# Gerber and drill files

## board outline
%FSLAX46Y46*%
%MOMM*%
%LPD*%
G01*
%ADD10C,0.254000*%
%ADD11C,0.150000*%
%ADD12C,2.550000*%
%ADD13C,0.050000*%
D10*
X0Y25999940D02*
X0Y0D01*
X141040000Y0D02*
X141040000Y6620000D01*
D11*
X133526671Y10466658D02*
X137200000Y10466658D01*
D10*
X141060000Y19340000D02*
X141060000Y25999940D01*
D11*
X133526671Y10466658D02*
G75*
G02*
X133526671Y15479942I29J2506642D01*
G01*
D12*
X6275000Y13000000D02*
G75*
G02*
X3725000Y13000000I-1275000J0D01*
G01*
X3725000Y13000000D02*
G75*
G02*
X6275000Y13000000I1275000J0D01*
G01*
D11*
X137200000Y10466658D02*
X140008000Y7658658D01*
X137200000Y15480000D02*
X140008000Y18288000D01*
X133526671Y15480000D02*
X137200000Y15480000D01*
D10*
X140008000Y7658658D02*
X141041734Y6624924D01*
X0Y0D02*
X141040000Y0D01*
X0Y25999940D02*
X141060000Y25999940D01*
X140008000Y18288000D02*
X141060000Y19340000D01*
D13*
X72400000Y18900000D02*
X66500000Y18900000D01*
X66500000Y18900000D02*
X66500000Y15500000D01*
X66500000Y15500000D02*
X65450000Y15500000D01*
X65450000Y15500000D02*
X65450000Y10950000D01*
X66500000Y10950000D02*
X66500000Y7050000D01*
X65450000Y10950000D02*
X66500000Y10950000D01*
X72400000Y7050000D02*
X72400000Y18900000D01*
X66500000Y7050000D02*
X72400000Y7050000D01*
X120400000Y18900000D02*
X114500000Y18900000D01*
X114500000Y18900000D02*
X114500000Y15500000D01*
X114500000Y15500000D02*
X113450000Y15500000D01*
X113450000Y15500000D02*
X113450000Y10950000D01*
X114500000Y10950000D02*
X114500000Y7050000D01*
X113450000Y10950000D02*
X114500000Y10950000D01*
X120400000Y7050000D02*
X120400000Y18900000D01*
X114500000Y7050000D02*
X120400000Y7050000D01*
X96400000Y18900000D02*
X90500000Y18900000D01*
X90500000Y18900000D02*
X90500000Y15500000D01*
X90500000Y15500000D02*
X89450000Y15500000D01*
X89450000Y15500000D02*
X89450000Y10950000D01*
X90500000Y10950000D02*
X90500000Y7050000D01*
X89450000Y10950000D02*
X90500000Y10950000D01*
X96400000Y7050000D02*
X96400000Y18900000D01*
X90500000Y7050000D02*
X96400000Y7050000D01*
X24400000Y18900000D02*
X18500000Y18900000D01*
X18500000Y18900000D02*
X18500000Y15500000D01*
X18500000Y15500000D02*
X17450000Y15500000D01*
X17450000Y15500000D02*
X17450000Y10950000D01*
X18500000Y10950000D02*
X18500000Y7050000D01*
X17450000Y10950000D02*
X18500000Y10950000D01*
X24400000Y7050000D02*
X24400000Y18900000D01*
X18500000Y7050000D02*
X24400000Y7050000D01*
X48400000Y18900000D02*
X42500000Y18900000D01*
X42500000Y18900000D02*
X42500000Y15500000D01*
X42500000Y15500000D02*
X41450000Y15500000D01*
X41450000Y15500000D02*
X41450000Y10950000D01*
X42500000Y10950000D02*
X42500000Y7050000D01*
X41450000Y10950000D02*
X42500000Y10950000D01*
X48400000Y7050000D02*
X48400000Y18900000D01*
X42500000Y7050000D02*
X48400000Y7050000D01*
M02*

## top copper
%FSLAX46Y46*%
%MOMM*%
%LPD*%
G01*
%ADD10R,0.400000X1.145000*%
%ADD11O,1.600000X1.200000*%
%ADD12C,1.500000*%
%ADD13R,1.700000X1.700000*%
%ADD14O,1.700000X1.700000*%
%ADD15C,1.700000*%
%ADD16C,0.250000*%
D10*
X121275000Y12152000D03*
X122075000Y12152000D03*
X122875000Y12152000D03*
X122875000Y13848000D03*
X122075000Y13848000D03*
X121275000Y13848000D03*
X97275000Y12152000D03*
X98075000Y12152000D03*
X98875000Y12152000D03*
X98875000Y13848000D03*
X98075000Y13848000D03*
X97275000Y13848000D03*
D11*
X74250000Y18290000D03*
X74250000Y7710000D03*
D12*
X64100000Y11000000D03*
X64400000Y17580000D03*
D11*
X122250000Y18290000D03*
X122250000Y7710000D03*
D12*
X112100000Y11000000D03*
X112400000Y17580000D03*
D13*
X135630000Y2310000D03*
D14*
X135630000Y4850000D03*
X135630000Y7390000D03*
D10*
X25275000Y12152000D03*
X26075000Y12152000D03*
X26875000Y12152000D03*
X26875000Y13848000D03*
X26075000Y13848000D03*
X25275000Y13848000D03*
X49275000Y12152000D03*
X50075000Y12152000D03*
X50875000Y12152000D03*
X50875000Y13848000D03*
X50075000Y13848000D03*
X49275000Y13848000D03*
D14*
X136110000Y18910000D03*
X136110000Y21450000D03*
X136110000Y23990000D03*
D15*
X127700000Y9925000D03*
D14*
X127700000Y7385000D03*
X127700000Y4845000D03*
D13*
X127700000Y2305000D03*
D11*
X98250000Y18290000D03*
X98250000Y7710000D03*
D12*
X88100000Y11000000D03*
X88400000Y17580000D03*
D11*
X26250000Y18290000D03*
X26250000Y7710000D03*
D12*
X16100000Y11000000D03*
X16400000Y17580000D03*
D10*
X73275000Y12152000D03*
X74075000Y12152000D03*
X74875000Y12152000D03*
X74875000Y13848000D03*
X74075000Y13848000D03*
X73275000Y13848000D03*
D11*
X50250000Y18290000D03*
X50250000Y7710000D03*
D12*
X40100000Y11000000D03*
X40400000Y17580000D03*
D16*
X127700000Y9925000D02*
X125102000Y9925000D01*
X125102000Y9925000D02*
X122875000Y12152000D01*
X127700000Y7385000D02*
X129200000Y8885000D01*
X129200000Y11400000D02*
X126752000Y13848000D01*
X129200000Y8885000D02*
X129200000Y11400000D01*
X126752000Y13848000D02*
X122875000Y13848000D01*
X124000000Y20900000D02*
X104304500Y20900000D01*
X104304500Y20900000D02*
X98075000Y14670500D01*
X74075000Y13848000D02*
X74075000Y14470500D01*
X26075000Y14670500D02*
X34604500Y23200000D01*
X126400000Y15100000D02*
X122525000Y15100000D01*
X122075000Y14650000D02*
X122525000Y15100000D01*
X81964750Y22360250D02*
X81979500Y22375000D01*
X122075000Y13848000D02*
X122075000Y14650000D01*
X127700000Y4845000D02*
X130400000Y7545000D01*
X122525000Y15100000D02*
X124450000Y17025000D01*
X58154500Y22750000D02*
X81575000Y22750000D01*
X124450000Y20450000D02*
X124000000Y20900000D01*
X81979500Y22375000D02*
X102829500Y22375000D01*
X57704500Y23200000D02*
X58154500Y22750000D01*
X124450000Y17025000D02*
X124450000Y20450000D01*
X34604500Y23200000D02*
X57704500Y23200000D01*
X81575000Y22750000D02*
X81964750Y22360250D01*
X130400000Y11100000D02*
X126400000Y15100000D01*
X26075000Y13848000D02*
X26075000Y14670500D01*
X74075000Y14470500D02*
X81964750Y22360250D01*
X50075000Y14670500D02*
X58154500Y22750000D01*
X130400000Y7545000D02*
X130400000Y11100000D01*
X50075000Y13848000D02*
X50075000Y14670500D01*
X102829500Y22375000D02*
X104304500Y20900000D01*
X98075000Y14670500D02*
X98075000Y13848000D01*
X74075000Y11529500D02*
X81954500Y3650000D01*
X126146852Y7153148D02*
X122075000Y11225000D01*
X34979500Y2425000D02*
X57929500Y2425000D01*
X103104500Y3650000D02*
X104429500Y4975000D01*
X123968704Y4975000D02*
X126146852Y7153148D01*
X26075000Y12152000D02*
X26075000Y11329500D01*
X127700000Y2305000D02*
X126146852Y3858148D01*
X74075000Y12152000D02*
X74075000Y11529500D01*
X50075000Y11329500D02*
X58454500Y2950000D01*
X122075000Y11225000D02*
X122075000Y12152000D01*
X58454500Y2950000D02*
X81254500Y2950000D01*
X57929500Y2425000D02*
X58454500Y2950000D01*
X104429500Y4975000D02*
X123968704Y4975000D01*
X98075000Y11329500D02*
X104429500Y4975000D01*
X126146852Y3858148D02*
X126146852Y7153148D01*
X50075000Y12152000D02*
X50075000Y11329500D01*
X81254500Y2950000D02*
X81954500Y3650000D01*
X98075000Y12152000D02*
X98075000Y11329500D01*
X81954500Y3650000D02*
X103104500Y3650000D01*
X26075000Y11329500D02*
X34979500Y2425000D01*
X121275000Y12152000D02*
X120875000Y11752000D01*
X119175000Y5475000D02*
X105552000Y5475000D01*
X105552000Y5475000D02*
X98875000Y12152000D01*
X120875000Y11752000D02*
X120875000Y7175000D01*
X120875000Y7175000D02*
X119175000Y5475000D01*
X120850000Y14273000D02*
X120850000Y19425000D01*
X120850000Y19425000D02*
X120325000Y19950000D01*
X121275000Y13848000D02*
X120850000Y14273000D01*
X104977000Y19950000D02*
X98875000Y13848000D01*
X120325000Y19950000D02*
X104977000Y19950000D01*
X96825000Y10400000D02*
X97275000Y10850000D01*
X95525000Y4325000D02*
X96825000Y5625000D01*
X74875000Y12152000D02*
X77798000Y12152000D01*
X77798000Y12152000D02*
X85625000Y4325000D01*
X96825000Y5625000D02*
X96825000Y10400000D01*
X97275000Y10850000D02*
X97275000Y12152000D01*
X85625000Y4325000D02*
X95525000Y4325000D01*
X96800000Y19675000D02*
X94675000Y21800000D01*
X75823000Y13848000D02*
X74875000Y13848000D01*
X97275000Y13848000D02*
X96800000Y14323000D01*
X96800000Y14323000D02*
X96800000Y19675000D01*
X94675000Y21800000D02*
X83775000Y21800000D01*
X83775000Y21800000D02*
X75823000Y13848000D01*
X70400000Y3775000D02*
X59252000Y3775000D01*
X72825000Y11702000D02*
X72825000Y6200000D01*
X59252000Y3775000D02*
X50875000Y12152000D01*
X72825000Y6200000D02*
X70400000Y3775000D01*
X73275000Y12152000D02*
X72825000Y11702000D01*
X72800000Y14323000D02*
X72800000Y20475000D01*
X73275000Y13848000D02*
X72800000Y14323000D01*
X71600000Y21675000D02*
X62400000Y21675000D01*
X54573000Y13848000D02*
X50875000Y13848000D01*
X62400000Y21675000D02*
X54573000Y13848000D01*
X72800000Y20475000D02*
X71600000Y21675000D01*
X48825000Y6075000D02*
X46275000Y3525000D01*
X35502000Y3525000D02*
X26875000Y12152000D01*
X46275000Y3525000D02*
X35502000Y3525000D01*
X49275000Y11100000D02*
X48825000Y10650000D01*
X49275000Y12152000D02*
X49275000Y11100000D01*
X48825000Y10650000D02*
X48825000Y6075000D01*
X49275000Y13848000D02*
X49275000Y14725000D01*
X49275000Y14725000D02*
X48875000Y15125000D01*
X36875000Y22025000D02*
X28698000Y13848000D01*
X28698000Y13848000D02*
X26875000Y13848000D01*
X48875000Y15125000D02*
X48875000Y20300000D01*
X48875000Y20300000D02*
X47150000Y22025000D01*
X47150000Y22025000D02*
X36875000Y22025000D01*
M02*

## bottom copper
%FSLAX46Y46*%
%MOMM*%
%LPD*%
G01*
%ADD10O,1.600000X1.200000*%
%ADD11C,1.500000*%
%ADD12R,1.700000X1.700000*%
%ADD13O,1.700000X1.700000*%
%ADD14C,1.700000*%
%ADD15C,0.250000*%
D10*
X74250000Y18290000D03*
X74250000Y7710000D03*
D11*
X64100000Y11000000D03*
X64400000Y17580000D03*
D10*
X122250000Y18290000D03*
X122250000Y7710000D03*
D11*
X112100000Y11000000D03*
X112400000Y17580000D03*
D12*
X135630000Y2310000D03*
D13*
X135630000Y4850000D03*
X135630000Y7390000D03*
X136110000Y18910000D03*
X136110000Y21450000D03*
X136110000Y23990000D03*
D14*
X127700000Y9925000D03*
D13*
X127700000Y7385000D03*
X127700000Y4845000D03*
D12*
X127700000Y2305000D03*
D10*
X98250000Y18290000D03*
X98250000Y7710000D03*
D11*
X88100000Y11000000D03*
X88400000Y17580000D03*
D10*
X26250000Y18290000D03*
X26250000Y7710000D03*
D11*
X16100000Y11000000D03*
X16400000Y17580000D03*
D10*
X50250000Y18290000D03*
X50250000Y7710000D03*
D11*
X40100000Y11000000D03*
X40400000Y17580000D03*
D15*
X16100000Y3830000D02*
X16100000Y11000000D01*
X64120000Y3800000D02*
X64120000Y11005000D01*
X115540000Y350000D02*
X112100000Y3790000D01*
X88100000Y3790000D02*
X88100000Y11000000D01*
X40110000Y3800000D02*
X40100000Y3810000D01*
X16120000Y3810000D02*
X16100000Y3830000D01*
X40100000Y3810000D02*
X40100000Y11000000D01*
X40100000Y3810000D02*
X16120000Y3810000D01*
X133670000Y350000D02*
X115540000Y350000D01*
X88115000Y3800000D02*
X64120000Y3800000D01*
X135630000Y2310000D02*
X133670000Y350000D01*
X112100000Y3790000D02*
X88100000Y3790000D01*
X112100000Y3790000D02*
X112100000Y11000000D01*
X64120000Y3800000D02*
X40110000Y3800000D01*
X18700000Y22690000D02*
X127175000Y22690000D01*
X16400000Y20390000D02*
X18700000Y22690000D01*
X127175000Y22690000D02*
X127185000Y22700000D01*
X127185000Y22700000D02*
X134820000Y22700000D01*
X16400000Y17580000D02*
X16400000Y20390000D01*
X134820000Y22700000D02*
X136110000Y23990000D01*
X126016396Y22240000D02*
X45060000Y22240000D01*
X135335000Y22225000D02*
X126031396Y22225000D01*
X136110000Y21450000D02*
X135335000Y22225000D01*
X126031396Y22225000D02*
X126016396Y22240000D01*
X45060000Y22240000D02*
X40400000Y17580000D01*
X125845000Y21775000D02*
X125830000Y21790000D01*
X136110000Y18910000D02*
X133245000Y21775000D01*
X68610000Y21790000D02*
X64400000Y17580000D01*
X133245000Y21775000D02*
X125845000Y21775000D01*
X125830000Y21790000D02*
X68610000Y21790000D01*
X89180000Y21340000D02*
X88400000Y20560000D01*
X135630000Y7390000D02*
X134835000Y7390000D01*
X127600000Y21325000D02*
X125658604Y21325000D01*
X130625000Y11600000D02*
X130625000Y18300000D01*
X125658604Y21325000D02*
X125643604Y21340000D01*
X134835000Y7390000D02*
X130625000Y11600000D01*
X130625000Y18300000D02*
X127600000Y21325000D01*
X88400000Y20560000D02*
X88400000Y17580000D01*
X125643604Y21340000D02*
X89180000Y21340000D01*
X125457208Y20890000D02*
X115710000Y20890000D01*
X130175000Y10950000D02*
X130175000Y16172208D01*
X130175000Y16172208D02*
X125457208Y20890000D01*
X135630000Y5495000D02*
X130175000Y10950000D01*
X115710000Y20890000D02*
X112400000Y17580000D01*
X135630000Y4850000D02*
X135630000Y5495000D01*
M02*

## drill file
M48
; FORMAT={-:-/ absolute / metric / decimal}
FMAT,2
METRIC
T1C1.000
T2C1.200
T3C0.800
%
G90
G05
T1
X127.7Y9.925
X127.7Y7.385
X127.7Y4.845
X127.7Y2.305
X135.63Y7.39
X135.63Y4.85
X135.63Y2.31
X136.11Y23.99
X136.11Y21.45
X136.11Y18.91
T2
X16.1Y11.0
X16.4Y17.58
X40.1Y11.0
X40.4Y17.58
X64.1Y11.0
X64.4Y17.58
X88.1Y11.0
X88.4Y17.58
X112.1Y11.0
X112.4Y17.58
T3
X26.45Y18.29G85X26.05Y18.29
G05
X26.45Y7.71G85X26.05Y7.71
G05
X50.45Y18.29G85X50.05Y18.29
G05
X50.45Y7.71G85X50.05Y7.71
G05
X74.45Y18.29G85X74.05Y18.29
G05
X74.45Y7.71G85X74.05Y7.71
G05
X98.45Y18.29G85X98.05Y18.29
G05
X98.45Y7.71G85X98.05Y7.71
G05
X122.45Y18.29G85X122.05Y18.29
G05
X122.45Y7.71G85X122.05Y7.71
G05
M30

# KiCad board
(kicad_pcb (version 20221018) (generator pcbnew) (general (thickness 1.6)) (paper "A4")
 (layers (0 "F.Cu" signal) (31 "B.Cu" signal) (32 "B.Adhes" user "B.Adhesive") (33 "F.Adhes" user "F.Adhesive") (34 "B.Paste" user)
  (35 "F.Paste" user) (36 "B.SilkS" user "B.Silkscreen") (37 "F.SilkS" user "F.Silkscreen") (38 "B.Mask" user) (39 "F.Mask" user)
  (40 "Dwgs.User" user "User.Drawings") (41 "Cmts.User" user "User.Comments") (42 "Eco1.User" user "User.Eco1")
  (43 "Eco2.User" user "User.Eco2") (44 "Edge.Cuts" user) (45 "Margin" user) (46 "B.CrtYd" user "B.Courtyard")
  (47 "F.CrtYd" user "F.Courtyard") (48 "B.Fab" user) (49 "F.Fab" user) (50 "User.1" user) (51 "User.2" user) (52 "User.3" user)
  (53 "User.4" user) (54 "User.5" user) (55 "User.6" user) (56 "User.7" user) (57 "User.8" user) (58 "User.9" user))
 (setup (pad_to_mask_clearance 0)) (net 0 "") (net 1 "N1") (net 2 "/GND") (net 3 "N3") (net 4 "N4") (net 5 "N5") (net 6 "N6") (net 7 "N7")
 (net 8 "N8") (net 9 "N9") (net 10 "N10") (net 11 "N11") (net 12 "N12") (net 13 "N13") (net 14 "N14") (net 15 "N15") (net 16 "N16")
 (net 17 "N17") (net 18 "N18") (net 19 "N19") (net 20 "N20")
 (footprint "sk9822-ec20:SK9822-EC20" (layer "F.Cu") (at 122.075 -13 90)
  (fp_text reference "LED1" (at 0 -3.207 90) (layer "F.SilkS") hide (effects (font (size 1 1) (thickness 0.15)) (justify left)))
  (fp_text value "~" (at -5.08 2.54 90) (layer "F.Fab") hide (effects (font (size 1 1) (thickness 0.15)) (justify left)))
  (pad "1" smd rect (at -0.848 -0.8 90) (size 1.145 0.4) (layers "F.Cu" "F.Paste" "F.Mask") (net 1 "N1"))
  (pad "2" smd rect (at -0.848 0 90) (size 1.145 0.4) (layers "F.Cu" "F.Paste" "F.Mask") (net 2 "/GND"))
  (pad "3" smd rect (at -0.848 0.8 90) (size 1.145 0.4) (layers "F.Cu" "F.Paste" "F.Mask") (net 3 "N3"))
  (pad "4" smd rect (at 0.848 0.8 90) (size 1.145 0.4) (layers "F.Cu" "F.Paste" "F.Mask") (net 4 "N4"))
  (pad "5" smd rect (at 0.848 0 90) (size 1.145 0.4) (layers "F.Cu" "F.Paste" "F.Mask") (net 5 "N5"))
  (pad "6" smd rect (at 0.848 -0.8 90) (size 1.145 0.4) (layers "F.Cu" "F.Paste" "F.Mask") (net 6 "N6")))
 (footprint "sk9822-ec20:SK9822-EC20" (layer "F.Cu") (at 98.075 -13 90)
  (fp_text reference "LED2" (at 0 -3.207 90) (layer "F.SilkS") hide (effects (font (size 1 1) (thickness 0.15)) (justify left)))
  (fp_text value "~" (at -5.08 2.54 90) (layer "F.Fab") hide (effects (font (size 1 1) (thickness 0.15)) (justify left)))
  (pad "1" smd rect (at -0.848 -0.8 90) (size 1.145 0.4) (layers "F.Cu" "F.Paste" "F.Mask") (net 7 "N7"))
  (pad "2" smd rect (at -0.848 0 90) (size 1.145 0.4) (layers "F.Cu" "F.Paste" "F.Mask") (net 2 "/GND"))
  (pad "3" smd rect (at -0.848 0.8 90) (size 1.145 0.4) (layers "F.Cu" "F.Paste" "F.Mask") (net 1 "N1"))
  (pad "4" smd rect (at 0.848 0.8 90) (size 1.145 0.4) (layers "F.Cu" "F.Paste" "F.Mask") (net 6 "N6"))
  (pad "5" smd rect (at 0.848 0 90) (size 1.145 0.4) (layers "F.Cu" "F.Paste" "F.Mask") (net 5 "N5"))
  (pad "6" smd rect (at 0.848 -0.8 90) (size 1.145 0.4) (layers "F.Cu" "F.Paste" "F.Mask") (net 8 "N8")))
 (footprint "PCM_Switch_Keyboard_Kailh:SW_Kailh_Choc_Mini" (layer "F.Cu") (at 69.5 -13 -90)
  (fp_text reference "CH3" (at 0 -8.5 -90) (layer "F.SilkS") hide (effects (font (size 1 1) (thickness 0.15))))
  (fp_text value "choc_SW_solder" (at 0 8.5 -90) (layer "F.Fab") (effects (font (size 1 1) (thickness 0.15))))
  (fp_line (start -5.9 -2.9) (end -5.9 3) (stroke (width 0.05) (type solid)) (layer "Edge.Cuts"))
  (fp_line (start -5.9 3) (end -2.5 3) (stroke (width 0.05) (type solid)) (layer "Edge.Cuts"))
  (fp_line (start -2.5 3) (end -2.5 4.05) (stroke (width 0.05) (type solid)) (layer "Edge.Cuts"))
  (fp_line (start -2.5 4.05) (end 2.05 4.05) (stroke (width 0.05) (type solid)) (layer "Edge.Cuts"))
  (fp_line (start 2.05 3) (end 5.95 3) (stroke (width 0.05) (type solid)) (layer "Edge.Cuts"))
  (fp_line (start 2.05 4.05) (end 2.05 3) (stroke (width 0.05) (type solid)) (layer "Edge.Cuts"))
  (fp_line (start 5.95 -2.9) (end -5.9 -2.9) (stroke (width 0.05) (type solid)) (layer "Edge.Cuts"))
  (fp_line (start 5.95 3) (end 5.95 -2.9) (stroke (width 0.05) (type solid)) (layer "Edge.Cuts"))
  (pad "" np_thru_hole oval (at -5.29 -4.75 270) (size 1.2 1.6) (drill oval 0.8 1.2) (layers "*.Cu" "*.Mask"))
  (pad "" np_thru_hole oval (at 5.29 -4.75 270) (size 1.2 1.6) (drill oval 0.8 1.2) (layers "*.Cu" "*.Mask"))
  (pad "1" thru_hole circle (at 2 5.4 270) (size 1.5 1.5) (drill 1.2) (layers "*.Cu" "*.Mask") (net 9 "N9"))
  (pad "2" thru_hole circle (at -4.58 5.1 270) (size 1.5 1.5) (drill 1.2) (layers "*.Cu" "*.Mask") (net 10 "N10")))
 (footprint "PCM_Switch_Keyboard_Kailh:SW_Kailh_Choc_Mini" (layer "F.Cu") (at 117.5 -13 -90)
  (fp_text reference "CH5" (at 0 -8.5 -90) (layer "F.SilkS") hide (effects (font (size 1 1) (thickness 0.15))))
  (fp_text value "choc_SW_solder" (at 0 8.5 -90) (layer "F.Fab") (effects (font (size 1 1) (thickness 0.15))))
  (fp_line (start -5.9 -2.9) (end -5.9 3) (stroke (width 0.05) (type solid)) (layer "Edge.Cuts"))
  (fp_line (start -5.9 3) (end -2.5 3) (stroke (width 0.05) (type solid)) (layer "Edge.Cuts"))
  (fp_line (start -2.5 3) (end -2.5 4.05) (stroke (width 0.05) (type solid)) (layer "Edge.Cuts"))
  (fp_line (start -2.5 4.05) (end 2.05 4.05) (stroke (width 0.05) (type solid)) (layer "Edge.Cuts"))
  (fp_line (start 2.05 3) (end 5.95 3) (stroke (width 0.05) (type solid)) (layer "Edge.Cuts"))
  (fp_line (start 2.05 4.05) (end 2.05 3) (stroke (width 0.05) (type solid)) (layer "Edge.Cuts"))
  (fp_line (start 5.95 -2.9) (end -5.9 -2.9) (stroke (width 0.05) (type solid)) (layer "Edge.Cuts"))
  (fp_line (start 5.95 3) (end 5.95 -2.9) (stroke (width 0.05) (type solid)) (layer "Edge.Cuts"))
  (pad "" np_thru_hole oval (at -5.29 -4.75 270) (size 1.2 1.6) (drill oval 0.8 1.2) (layers "*.Cu" "*.Mask"))
  (pad "" np_thru_hole oval (at 5.29 -4.75 270) (size 1.2 1.6) (drill oval 0.8 1.2) (layers "*.Cu" "*.Mask"))
  (pad "1" thru_hole circle (at 2 5.4 270) (size 1.5 1.5) (drill 1.2) (layers "*.Cu" "*.Mask") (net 9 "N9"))
  (pad "2" thru_hole circle (at -4.58 5.1 270) (size 1.5 1.5) (drill 1.2) (layers "*.Cu" "*.Mask") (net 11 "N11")))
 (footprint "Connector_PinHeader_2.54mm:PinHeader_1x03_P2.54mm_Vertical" (layer "F.Cu") (at 135.63 -2.31 180)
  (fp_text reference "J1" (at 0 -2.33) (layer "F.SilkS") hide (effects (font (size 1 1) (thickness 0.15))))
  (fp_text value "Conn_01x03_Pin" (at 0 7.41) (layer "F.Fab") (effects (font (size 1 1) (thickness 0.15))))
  (pad "1" thru_hole rect (at 0 0 180) (size 1.7 1.7) (drill 1) (layers "*.Cu" "*.Mask") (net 9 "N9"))
  (pad "2" thru_hole oval (at 0 2.54 180) (size 1.7 1.7) (drill 1) (layers "*.Cu" "*.Mask") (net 11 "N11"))
  (pad "3" thru_hole oval (at 0 5.08 180) (size 1.7 1.7) (drill 1) (layers "*.Cu" "*.Mask") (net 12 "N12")))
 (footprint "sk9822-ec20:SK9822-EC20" (layer "F.Cu") (at 26.075 -13 90)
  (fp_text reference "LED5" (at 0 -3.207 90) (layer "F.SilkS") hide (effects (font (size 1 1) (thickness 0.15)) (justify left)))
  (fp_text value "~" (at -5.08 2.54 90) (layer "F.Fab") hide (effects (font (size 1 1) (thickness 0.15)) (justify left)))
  (pad "1" smd rect (at -0.848 -0.8 90) (size 1.145 0.4) (layers "F.Cu" "F.Paste" "F.Mask") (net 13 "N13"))
  (pad "2" smd rect (at -0.848 0 90) (size 1.145 0.4) (layers "F.Cu" "F.Paste" "F.Mask") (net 2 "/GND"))
  (pad "3" smd rect (at -0.848 0.8 90) (size 1.145 0.4) (layers "F.Cu" "F.Paste" "F.Mask") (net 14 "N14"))
  (pad "4" smd rect (at 0.848 0.8 90) (size 1.145 0.4) (layers "F.Cu" "F.Paste" "F.Mask") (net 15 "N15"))
  (pad "5" smd rect (at 0.848 0 90) (size 1.145 0.4) (layers "F.Cu" "F.Paste" "F.Mask") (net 5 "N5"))
  (pad "6" smd rect (at 0.848 -0.8 90) (size 1.145 0.4) (layers "F.Cu" "F.Paste" "F.Mask") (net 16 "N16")))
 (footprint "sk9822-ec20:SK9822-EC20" (layer "F.Cu") (at 50.075 -13 90)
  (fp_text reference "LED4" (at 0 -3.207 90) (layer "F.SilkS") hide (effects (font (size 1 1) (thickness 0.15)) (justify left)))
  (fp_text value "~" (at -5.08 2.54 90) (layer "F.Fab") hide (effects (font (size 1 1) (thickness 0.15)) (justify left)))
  (pad "1" smd rect (at -0.848 -0.8 90) (size 1.145 0.4) (layers "F.Cu" "F.Paste" "F.Mask") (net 14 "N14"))
  (pad "2" smd rect (at -0.848 0 90) (size 1.145 0.4) (layers "F.Cu" "F.Paste" "F.Mask") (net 2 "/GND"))
  (pad "3" smd rect (at -0.848 0.8 90) (size 1.145 0.4) (layers "F.Cu" "F.Paste" "F.Mask") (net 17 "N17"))
  (pad "4" smd rect (at 0.848 0.8 90) (size 1.145 0.4) (layers "F.Cu" "F.Paste" "F.Mask") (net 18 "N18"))
  (pad "5" smd rect (at 0.848 0 90) (size 1.145 0.4) (layers "F.Cu" "F.Paste" "F.Mask") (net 5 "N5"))
  (pad "6" smd rect (at 0.848 -0.8 90) (size 1.145 0.4) (layers "F.Cu" "F.Paste" "F.Mask") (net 15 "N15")))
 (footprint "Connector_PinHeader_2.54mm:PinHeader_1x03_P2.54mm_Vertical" (layer "F.Cu") (at 136.11 -18.91 180)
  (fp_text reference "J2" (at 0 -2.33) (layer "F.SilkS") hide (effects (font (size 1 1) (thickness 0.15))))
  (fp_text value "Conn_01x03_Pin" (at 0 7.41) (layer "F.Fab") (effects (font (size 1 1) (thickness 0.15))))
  (pad "1" thru_hole oval (at 0 0 180) (size 1.7 1.7) (drill 1) (layers "*.Cu" "*.Mask") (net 10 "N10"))
  (pad "2" thru_hole oval (at 0 2.54 180) (size 1.7 1.7) (drill 1) (layers "*.Cu" "*.Mask") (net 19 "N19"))
  (pad "3" thru_hole oval (at 0 5.08 180) (size 1.7 1.7) (drill 1) (layers "*.Cu" "*.Mask") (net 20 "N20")))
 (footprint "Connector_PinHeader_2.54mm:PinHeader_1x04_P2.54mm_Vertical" (layer "F.Cu") (at 127.7 -9.925)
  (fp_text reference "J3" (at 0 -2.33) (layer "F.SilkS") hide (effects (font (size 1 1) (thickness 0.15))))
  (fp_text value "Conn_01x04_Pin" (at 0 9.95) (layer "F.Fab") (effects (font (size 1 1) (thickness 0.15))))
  (pad "1" thru_hole circle (at 0 0) (size 1.7 1.7) (drill 1) (layers "*.Cu" "*.Mask") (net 3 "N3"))
  (pad "2" thru_hole oval (at 0 2.54) (size 1.7 1.7) (drill 1) (layers "*.Cu" "*.Mask") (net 4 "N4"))
  (pad "3" thru_hole oval (at 0 5.08) (size 1.7 1.7) (drill 1) (layers "*.Cu" "*.Mask") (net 5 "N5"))
  (pad "4" thru_hole rect (at 0 7.62) (size 1.7 1.7) (drill 1) (layers "*.Cu" "*.Mask") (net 2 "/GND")))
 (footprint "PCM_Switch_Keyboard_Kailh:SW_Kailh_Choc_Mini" (layer "F.Cu") (at 93.5 -13 -90)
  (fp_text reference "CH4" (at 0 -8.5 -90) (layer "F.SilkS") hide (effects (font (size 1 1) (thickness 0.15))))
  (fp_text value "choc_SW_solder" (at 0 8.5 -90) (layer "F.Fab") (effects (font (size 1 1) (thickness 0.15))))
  (fp_line (start -5.9 -2.9) (end -5.9 3) (stroke (width 0.05) (type solid)) (layer "Edge.Cuts"))
  (fp_line (start -5.9 3) (end -2.5 3) (stroke (width 0.05) (type solid)) (layer "Edge.Cuts"))
  (fp_line (start -2.5 3) (end -2.5 4.05) (stroke (width 0.05) (type solid)) (layer "Edge.Cuts"))
  (fp_line (start -2.5 4.05) (end 2.05 4.05) (stroke (width 0.05) (type solid)) (layer "Edge.Cuts"))
  (fp_line (start 2.05 3) (end 5.95 3) (stroke (width 0.05) (type solid)) (layer "Edge.Cuts"))
  (fp_line (start 2.05 4.05) (end 2.05 3) (stroke (width 0.05) (type solid)) (layer "Edge.Cuts"))
  (fp_line (start 5.95 -2.9) (end -5.9 -2.9) (stroke (width 0.05) (type solid)) (layer "Edge.Cuts"))
  (fp_line (start 5.95 3) (end 5.95 -2.9) (stroke (width 0.05) (type solid)) (layer "Edge.Cuts"))
  (pad "" np_thru_hole oval (at -5.29 -4.75 270) (size 1.2 1.6) (drill oval 0.8 1.2) (layers "*.Cu" "*.Mask"))
  (pad "" np_thru_hole oval (at 5.29 -4.75 270) (size 1.2 1.6) (drill oval 0.8 1.2) (layers "*.Cu" "*.Mask"))
  (pad "1" thru_hole circle (at 2 5.4 270) (size 1.5 1.5) (drill 1.2) (layers "*.Cu" "*.Mask") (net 9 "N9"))
  (pad "2" thru_hole circle (at -4.58 5.1 270) (size 1.5 1.5) (drill 1.2) (layers "*.Cu" "*.Mask") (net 12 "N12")))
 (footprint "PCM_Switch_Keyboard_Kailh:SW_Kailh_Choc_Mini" (layer "F.Cu") (at 21.5 -13 -90)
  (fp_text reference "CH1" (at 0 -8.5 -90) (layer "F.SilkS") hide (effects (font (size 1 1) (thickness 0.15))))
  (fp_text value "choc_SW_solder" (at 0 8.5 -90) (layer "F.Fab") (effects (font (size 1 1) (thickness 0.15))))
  (fp_line (start -5.9 -2.9) (end -5.9 3) (stroke (width 0.05) (type solid)) (layer "Edge.Cuts"))
  (fp_line (start -5.9 3) (end -2.5 3) (stroke (width 0.05) (type solid)) (layer "Edge.Cuts"))
  (fp_line (start -2.5 3) (end -2.5 4.05) (stroke (width 0.05) (type solid)) (layer "Edge.Cuts"))
  (fp_line (start -2.5 4.05) (end 2.05 4.05) (stroke (width 0.05) (type solid)) (layer "Edge.Cuts"))
  (fp_line (start 2.05 3) (end 5.95 3) (stroke (width 0.05) (type solid)) (layer "Edge.Cuts"))
  (fp_line (start 2.05 4.05) (end 2.05 3) (stroke (width 0.05) (type solid)) (layer "Edge.Cuts"))
  (fp_line (start 5.95 -2.9) (end -5.9 -2.9) (stroke (width 0.05) (type solid)) (layer "Edge.Cuts"))
  (fp_line (start 5.95 3) (end 5.95 -2.9) (stroke (width 0.05) (type solid)) (layer "Edge.Cuts"))
  (pad "" np_thru_hole oval (at -5.29 -4.75 270) (size 1.2 1.6) (drill oval 0.8 1.2) (layers "*.Cu" "*.Mask"))
  (pad "" np_thru_hole oval (at 5.29 -4.75 270) (size 1.2 1.6) (drill oval 0.8 1.2) (layers "*.Cu" "*.Mask"))
  (pad "1" thru_hole circle (at 2 5.4 270) (size 1.5 1.5) (drill 1.2) (layers "*.Cu" "*.Mask") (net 9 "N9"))
  (pad "2" thru_hole circle (at -4.58 5.1 270) (size 1.5 1.5) (drill 1.2) (layers "*.Cu" "*.Mask") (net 20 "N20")))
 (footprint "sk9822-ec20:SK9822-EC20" (layer "F.Cu") (at 74.075 -13 90)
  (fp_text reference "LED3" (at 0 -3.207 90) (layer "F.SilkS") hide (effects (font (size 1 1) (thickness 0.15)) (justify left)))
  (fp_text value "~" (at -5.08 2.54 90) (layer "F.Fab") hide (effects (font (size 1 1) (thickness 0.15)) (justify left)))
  (pad "1" smd rect (at -0.848 -0.8 90) (size 1.145 0.4) (layers "F.Cu" "F.Paste" "F.Mask") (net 17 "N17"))
  (pad "2" smd rect (at -0.848 0 90) (size 1.145 0.4) (layers "F.Cu" "F.Paste" "F.Mask") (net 2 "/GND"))
  (pad "3" smd rect (at -0.848 0.8 90) (size 1.145 0.4) (layers "F.Cu" "F.Paste" "F.Mask") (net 7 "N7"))
  (pad "4" smd rect (at 0.848 0.8 90) (size 1.145 0.4) (layers "F.Cu" "F.Paste" "F.Mask") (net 8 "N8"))
  (pad "5" smd rect (at 0.848 0 90) (size 1.145 0.4) (layers "F.Cu" "F.Paste" "F.Mask") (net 5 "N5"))
  (pad "6" smd rect (at 0.848 -0.8 90) (size 1.145 0.4) (layers "F.Cu" "F.Paste" "F.Mask") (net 18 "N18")))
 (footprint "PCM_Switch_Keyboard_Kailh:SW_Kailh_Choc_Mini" (layer "F.Cu") (at 45.5 -13 -90)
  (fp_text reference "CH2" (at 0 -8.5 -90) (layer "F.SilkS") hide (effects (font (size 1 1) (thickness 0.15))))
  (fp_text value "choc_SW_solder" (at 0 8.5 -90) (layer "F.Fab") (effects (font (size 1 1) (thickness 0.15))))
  (fp_line (start -5.9 -2.9) (end -5.9 3) (stroke (width 0.05) (type solid)) (layer "Edge.Cuts"))
  (fp_line (start -5.9 3) (end -2.5 3) (stroke (width 0.05) (type solid)) (layer "Edge.Cuts"))
  (fp_line (start -2.5 3) (end -2.5 4.05) (stroke (width 0.05) (type solid)) (layer "Edge.Cuts"))
  (fp_line (start -2.5 4.05) (end 2.05 4.05) (stroke (width 0.05) (type solid)) (layer "Edge.Cuts"))
  (fp_line (start 2.05 3) (end 5.95 3) (stroke (width 0.05) (type solid)) (layer "Edge.Cuts"))
  (fp_line (start 2.05 4.05) (end 2.05 3) (stroke (width 0.05) (type solid)) (layer "Edge.Cuts"))
  (fp_line (start 5.95 -2.9) (end -5.9 -2.9) (stroke (width 0.05) (type solid)) (layer "Edge.Cuts"))
  (fp_line (start 5.95 3) (end 5.95 -2.9) (stroke (width 0.05) (type solid)) (layer "Edge.Cuts"))
  (pad "" np_thru_hole oval (at -5.29 -4.75 270) (size 1.2 1.6) (drill oval 0.8 1.2) (layers "*.Cu" "*.Mask"))
  (pad "" np_thru_hole oval (at 5.29 -4.75 270) (size 1.2 1.6) (drill oval 0.8 1.2) (layers "*.Cu" "*.Mask"))
  (pad "1" thru_hole circle (at 2 5.4 270) (size 1.5 1.5) (drill 1.2) (layers "*.Cu" "*.Mask") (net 9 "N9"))
  (pad "2" thru_hole circle (at -4.58 5.1 270) (size 1.5 1.5) (drill 1.2) (layers "*.Cu" "*.Mask") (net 19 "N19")))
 (gr_line (start 0 -25.99994) (end 0 0) (stroke (width 0.254) (type solid)) (layer "Edge.Cuts"))
 (gr_line (start 141.04 0) (end 141.04 -6.62) (stroke (width 0.254) (type solid)) (layer "Edge.Cuts"))
 (gr_line (start 133.526671 -10.466658) (end 137.2 -10.466658) (stroke (width 0.15) (type default)) (layer "Edge.Cuts"))
 (gr_line (start 141.06 -19.34) (end 141.06 -25.99994) (stroke (width 0.254) (type solid)) (layer "Edge.Cuts"))
 (gr_arc (start 133.526671 -10.466658) (mid 131.02 -12.973329) (end 133.526671 -15.48) (stroke (width 0.15) (type default))
  (layer "Edge.Cuts"))
 (gr_circle (center 5 -13) (end 7.5 -13) (stroke (width 0.1) (type solid)) (fill solid) (layer "Edge.Cuts"))
 (gr_line (start 137.2 -10.466658) (end 140.008 -7.658658) (stroke (width 0.15) (type default)) (layer "Edge.Cuts"))
 (gr_line (start 137.2 -15.48) (end 140.008 -18.288) (stroke (width 0.15) (type default)) (layer "Edge.Cuts"))
 (gr_line (start 133.526671 -15.48) (end 137.2 -15.48) (stroke (width 0.15) (type default)) (layer "Edge.Cuts"))
 (gr_line (start 140.008 -7.658658) (end 141.041734 -6.624924) (stroke (width 0.254) (type solid)) (layer "Edge.Cuts"))
 (gr_line (start 0 0) (end 141.04 0) (stroke (width 0.254) (type solid)) (layer "Edge.Cuts"))
 (gr_line (start 0 -25.99994) (end 141.06 -25.99994) (stroke (width 0.254) (type solid)) (layer "Edge.Cuts"))
 (gr_line (start 140.008 -18.288) (end 141.06 -19.34) (stroke (width 0.254) (type solid)) (layer "Edge.Cuts"))
 (segment (start 16.1 -3.83) (end 16.1 -11) (width 0.25) (layer "B.Cu") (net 9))
 (segment (start 64.12 -3.8) (end 64.12 -11.005) (width 0.25) (layer "B.Cu") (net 9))
 (segment (start 115.54 -0.35) (end 112.1 -3.79) (width 0.25) (layer "B.Cu") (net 9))
 (segment (start 88.1 -3.79) (end 88.1 -11) (width 0.25) (layer "B.Cu") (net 9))
 (segment (start 40.11 -3.8) (end 40.1 -3.81) (width 0.25) (layer "B.Cu") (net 9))
 (segment (start 16.12 -3.81) (end 16.1 -3.83) (width 0.25) (layer "B.Cu") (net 9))
 (segment (start 40.1 -3.81) (end 40.1 -11) (width 0.25) (layer "B.Cu") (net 9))
 (segment (start 40.1 -3.81) (end 16.12 -3.81) (width 0.25) (layer "B.Cu") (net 9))
 (segment (start 133.67 -0.35) (end 115.54 -0.35) (width 0.25) (layer "B.Cu") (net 9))
 (segment (start 88.115 -3.8) (end 64.12 -3.8) (width 0.25) (layer "B.Cu") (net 9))
 (segment (start 135.63 -2.31) (end 133.67 -0.35) (width 0.25) (layer "B.Cu") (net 9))
 (segment (start 112.1 -3.79) (end 88.1 -3.79) (width 0.25) (layer "B.Cu") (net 9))
 (segment (start 112.1 -3.79) (end 112.1 -11) (width 0.25) (layer "B.Cu") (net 9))
 (segment (start 64.12 -3.8) (end 40.11 -3.8) (width 0.25) (layer "B.Cu") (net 9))
 (segment (start 18.7 -22.69) (end 127.175 -22.69) (width 0.25) (layer "B.Cu") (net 20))
 (segment (start 16.4 -20.39) (end 18.7 -22.69) (width 0.25) (layer "B.Cu") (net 20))
 (segment (start 127.175 -22.69) (end 127.185 -22.7) (width 0.25) (layer "B.Cu") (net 20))
 (segment (start 127.185 -22.7) (end 134.82 -22.7) (width 0.25) (layer "B.Cu") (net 20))
 (segment (start 16.4 -17.58) (end 16.4 -20.39) (width 0.25) (layer "B.Cu") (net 20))
 (segment (start 134.82 -22.7) (end 136.11 -23.99) (width 0.25) (layer "B.Cu") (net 20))
 (segment (start 126.016396 -22.24) (end 45.06 -22.24) (width 0.25) (layer "B.Cu") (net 19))
 (segment (start 135.335 -22.225) (end 126.031396 -22.225) (width 0.25) (layer "B.Cu") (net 19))
 (segment (start 136.11 -21.45) (end 135.335 -22.225) (width 0.25) (layer "B.Cu") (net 19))
 (segment (start 126.031396 -22.225) (end 126.016396 -22.24) (width 0.25) (layer "B.Cu") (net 19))
 (segment (start 45.06 -22.24) (end 40.4 -17.58) (width 0.25) (layer "B.Cu") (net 19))
 (segment (start 125.845 -21.775) (end 125.83 -21.79) (width 0.25) (layer "B.Cu") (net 10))
 (segment (start 136.11 -18.91) (end 133.245 -21.775) (width 0.25) (layer "B.Cu") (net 10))
 (segment (start 68.61 -21.79) (end 64.4 -17.58) (width 0.25) (layer "B.Cu") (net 10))
 (segment (start 133.245 -21.775) (end 125.845 -21.775) (width 0.25) (layer "B.Cu") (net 10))
 (segment (start 125.83 -21.79) (end 68.61 -21.79) (width 0.25) (layer "B.Cu") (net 10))
 (segment (start 89.18 -21.34) (end 88.4 -20.56) (width 0.25) (layer "B.Cu") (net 12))
 (segment (start 135.63 -7.39) (end 134.835 -7.39) (width 0.25) (layer "B.Cu") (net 12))
 (segment (start 127.6 -21.325) (end 125.658604 -21.325) (width 0.25) (layer "B.Cu") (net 12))
 (segment (start 130.625 -11.6) (end 130.625 -18.3) (width 0.25) (layer "B.Cu") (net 12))
 (segment (start 125.658604 -21.325) (end 125.643604 -21.34) (width 0.25) (layer "B.Cu") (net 12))
 (segment (start 134.835 -7.39) (end 130.625 -11.6) (width 0.25) (layer "B.Cu") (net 12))
 (segment (start 130.625 -18.3) (end 127.6 -21.325) (width 0.25) (layer "B.Cu") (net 12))
 (segment (start 88.4 -20.56) (end 88.4 -17.58) (width 0.25) (layer "B.Cu") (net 12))
 (segment (start 125.643604 -21.34) (end 89.18 -21.34) (width 0.25) (layer "B.Cu") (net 12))
 (segment (start 125.457208 -20.89) (end 115.71 -20.89) (width 0.25) (layer "B.Cu") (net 11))
 (segment (start 130.175 -10.95) (end 130.175 -16.172208) (width 0.25) (layer "B.Cu") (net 11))
 (segment (start 130.175 -16.172208) (end 125.457208 -20.89) (width 0.25) (layer "B.Cu") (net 11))
 (segment (start 135.63 -5.495) (end 130.175 -10.95) (width 0.25) (layer "B.Cu") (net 11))
 (segment (start 115.71 -20.89) (end 112.4 -17.58) (width 0.25) (layer "B.Cu") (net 11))
 (segment (start 135.63 -4.85) (end 135.63 -5.495) (width 0.25) (layer "B.Cu") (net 11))
 (segment (start 127.7 -9.925) (end 125.102 -9.925) (width 0.25) (layer "F.Cu") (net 3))
 (segment (start 125.102 -9.925) (end 122.875 -12.152) (width 0.25) (layer "F.Cu") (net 3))
 (segment (start 127.7 -7.385) (end 129.2 -8.885) (width 0.25) (layer "F.Cu") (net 4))
 (segment (start 129.2 -11.4) (end 126.752 -13.848) (width 0.25) (layer "F.Cu") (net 4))
 (segment (start 129.2 -8.885) (end 129.2 -11.4) (width 0.25) (layer "F.Cu") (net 4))
 (segment (start 126.752 -13.848) (end 122.875 -13.848) (width 0.25) (layer "F.Cu") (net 4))
 (segment (start 124 -20.9) (end 104.3045 -20.9) (width 0.25) (layer "F.Cu") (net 5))
 (segment (start 104.3045 -20.9) (end 98.075 -14.6705) (width 0.25) (layer "F.Cu") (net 5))
 (segment (start 74.075 -13.848) (end 74.075 -14.4705) (width 0.25) (layer "F.Cu") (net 5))
 (segment (start 26.075 -14.6705) (end 34.6045 -23.2) (width 0.25) (layer "F.Cu") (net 5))
 (segment (start 126.4 -15.1) (end 122.525 -15.1) (width 0.25) (layer "F.Cu") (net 5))
 (segment (start 122.075 -14.65) (end 122.525 -15.1) (width 0.25) (layer "F.Cu") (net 5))
 (segment (start 81.96475 -22.36025) (end 81.9795 -22.375) (width 0.25) (layer "F.Cu") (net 5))
 (segment (start 122.075 -13.848) (end 122.075 -14.65) (width 0.25) (layer "F.Cu") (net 5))
 (segment (start 127.7 -4.845) (end 130.4 -7.545) (width 0.25) (layer "F.Cu") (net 5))
 (segment (start 122.525 -15.1) (end 124.45 -17.025) (width 0.25) (layer "F.Cu") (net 5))
 (segment (start 58.1545 -22.75) (end 81.575 -22.75) (width 0.25) (layer "F.Cu") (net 5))
 (segment (start 124.45 -20.45) (end 124 -20.9) (width 0.25) (layer "F.Cu") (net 5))
 (segment (start 81.9795 -22.375) (end 102.8295 -22.375) (width 0.25) (layer "F.Cu") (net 5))
 (segment (start 57.7045 -23.2) (end 58.1545 -22.75) (width 0.25) (layer "F.Cu") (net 5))
 (segment (start 124.45 -17.025) (end 124.45 -20.45) (width 0.25) (layer "F.Cu") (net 5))
 (segment (start 34.6045 -23.2) (end 57.7045 -23.2) (width 0.25) (layer "F.Cu") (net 5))
 (segment (start 81.575 -22.75) (end 81.96475 -22.36025) (width 0.25) (layer "F.Cu") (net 5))
 (segment (start 130.4 -11.1) (end 126.4 -15.1) (width 0.25) (layer "F.Cu") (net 5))
 (segment (start 26.075 -13.848) (end 26.075 -14.6705) (width 0.25) (layer "F.Cu") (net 5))
 (segment (start 74.075 -14.4705) (end 81.96475 -22.36025) (width 0.25) (layer "F.Cu") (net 5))
 (segment (start 50.075 -14.6705) (end 58.1545 -22.75) (width 0.25) (layer "F.Cu") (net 5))
 (segment (start 130.4 -7.545) (end 130.4 -11.1) (width 0.25) (layer "F.Cu") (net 5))
 (segment (start 50.075 -13.848) (end 50.075 -14.6705) (width 0.25) (layer "F.Cu") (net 5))
 (segment (start 102.8295 -22.375) (end 104.3045 -20.9) (width 0.25) (layer "F.Cu") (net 5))
 (segment (start 98.075 -14.6705) (end 98.075 -13.848) (width 0.25) (layer "F.Cu") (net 5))
 (segment (start 74.075 -11.5295) (end 81.9545 -3.65) (width 0.25) (layer "F.Cu") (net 2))
 (segment (start 126.146852 -7.153148) (end 122.075 -11.225) (width 0.25) (layer "F.Cu") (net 2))
 (segment (start 34.9795 -2.425) (end 57.9295 -2.425) (width 0.25) (layer "F.Cu") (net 2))
 (segment (start 103.1045 -3.65) (end 104.4295 -4.975) (width 0.25) (layer "F.Cu") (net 2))
 (segment (start 123.968704 -4.975) (end 126.146852 -7.153148) (width 0.25) (layer "F.Cu") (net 2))
 (segment (start 26.075 -12.152) (end 26.075 -11.3295) (width 0.25) (layer "F.Cu") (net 2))
 (segment (start 127.7 -2.305) (end 126.146852 -3.858148) (width 0.25) (layer "F.Cu") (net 2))
 (segment (start 74.075 -12.152) (end 74.075 -11.5295) (width 0.25) (layer "F.Cu") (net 2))
 (segment (start 50.075 -11.3295) (end 58.4545 -2.95) (width 0.25) (layer "F.Cu") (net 2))
 (segment (start 122.075 -11.225) (end 122.075 -12.152) (width 0.25) (layer "F.Cu") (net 2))
 (segment (start 58.4545 -2.95) (end 81.2545 -2.95) (width 0.25) (layer "F.Cu") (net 2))
 (segment (start 57.9295 -2.425) (end 58.4545 -2.95) (width 0.25) (layer "F.Cu") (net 2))
 (segment (start 104.4295 -4.975) (end 123.968704 -4.975) (width 0.25) (layer "F.Cu") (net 2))
 (segment (start 98.075 -11.3295) (end 104.4295 -4.975) (width 0.25) (layer "F.Cu") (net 2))
 (segment (start 126.146852 -3.858148) (end 126.146852 -7.153148) (width 0.25) (layer "F.Cu") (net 2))
 (segment (start 50.075 -12.152) (end 50.075 -11.3295) (width 0.25) (layer "F.Cu") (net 2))
 (segment (start 81.2545 -2.95) (end 81.9545 -3.65) (width 0.25) (layer "F.Cu") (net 2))
 (segment (start 98.075 -12.152) (end 98.075 -11.3295) (width 0.25) (layer "F.Cu") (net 2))
 (segment (start 81.9545 -3.65) (end 103.1045 -3.65) (width 0.25) (layer "F.Cu") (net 2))
 (segment (start 26.075 -11.3295) (end 34.9795 -2.425) (width 0.25) (layer "F.Cu") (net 2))
 (segment (start 121.275 -12.152) (end 120.875 -11.752) (width 0.25) (layer "F.Cu") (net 1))
 (segment (start 119.175 -5.475) (end 105.552 -5.475) (width 0.25) (layer "F.Cu") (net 1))
 (segment (start 105.552 -5.475) (end 98.875 -12.152) (width 0.25) (layer "F.Cu") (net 1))
 (segment (start 120.875 -11.752) (end 120.875 -7.175) (width 0.25) (layer "F.Cu") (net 1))
 (segment (start 120.875 -7.175) (end 119.175 -5.475) (width 0.25) (layer "F.Cu") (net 1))
 (segment (start 120.85 -14.273) (end 120.85 -19.425) (width 0.25) (layer "F.Cu") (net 6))
 (segment (start 120.85 -19.425) (end 120.325 -19.95) (width 0.25) (layer "F.Cu") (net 6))
 (segment (start 121.275 -13.848) (end 120.85 -14.273) (width 0.25) (layer "F.Cu") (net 6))
 (segment (start 104.977 -19.95) (end 98.875 -13.848) (width 0.25) (layer "F.Cu") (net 6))
 (segment (start 120.325 -19.95) (end 104.977 -19.95) (width 0.25) (layer "F.Cu") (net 6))
 (segment (start 96.825 -10.4) (end 97.275 -10.85) (width 0.25) (layer "F.Cu") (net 7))
 (segment (start 95.525 -4.325) (end 96.825 -5.625) (width 0.25) (layer "F.Cu") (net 7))
 (segment (start 74.875 -12.152) (end 77.798 -12.152) (width 0.25) (layer "F.Cu") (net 7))
 (segment (start 77.798 -12.152) (end 85.625 -4.325) (width 0.25) (layer "F.Cu") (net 7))
 (segment (start 96.825 -5.625) (end 96.825 -10.4) (width 0.25) (layer "F.Cu") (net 7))
 (segment (start 97.275 -10.85) (end 97.275 -12.152) (width 0.25) (layer "F.Cu") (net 7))
 (segment (start 85.625 -4.325) (end 95.525 -4.325) (width 0.25) (layer "F.Cu") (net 7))
 (segment (start 96.8 -19.675) (end 94.675 -21.8) (width 0.25) (layer "F.Cu") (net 8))
 (segment (start 75.823 -13.848) (end 74.875 -13.848) (width 0.25) (layer "F.Cu") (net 8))
 (segment (start 97.275 -13.848) (end 96.8 -14.323) (width 0.25) (layer "F.Cu") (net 8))
 (segment (start 96.8 -14.323) (end 96.8 -19.675) (width 0.25) (layer "F.Cu") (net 8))
 (segment (start 94.675 -21.8) (end 83.775 -21.8) (width 0.25) (layer "F.Cu") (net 8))
 (segment (start 83.775 -21.8) (end 75.823 -13.848) (width 0.25) (layer "F.Cu") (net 8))
 (segment (start 70.4 -3.775) (end 59.252 -3.775) (width 0.25) (layer "F.Cu") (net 17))
 (segment (start 72.825 -11.702) (end 72.825 -6.2) (width 0.25) (layer "F.Cu") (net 17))
 (segment (start 59.252 -3.775) (end 50.875 -12.152) (width 0.25) (layer "F.Cu") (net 17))
 (segment (start 72.825 -6.2) (end 70.4 -3.775) (width 0.25) (layer "F.Cu") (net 17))
 (segment (start 73.275 -12.152) (end 72.825 -11.702) (width 0.25) (layer "F.Cu") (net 17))
 (segment (start 72.8 -14.323) (end 72.8 -20.475) (width 0.25) (layer "F.Cu") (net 18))
 (segment (start 73.275 -13.848) (end 72.8 -14.323) (width 0.25) (layer "F.Cu") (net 18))
 (segment (start 71.6 -21.675) (end 62.4 -21.675) (width 0.25) (layer "F.Cu") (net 18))
 (segment (start 54.573 -13.848) (end 50.875 -13.848) (width 0.25) (layer "F.Cu") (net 18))
 (segment (start 62.4 -21.675) (end 54.573 -13.848) (width 0.25) (layer "F.Cu") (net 18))
 (segment (start 72.8 -20.475) (end 71.6 -21.675) (width 0.25) (layer "F.Cu") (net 18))
 (segment (start 48.825 -6.075) (end 46.275 -3.525) (width 0.25) (layer "F.Cu") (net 14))
 (segment (start 35.502 -3.525) (end 26.875 -12.152) (width 0.25) (layer "F.Cu") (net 14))
 (segment (start 46.275 -3.525) (end 35.502 -3.525) (width 0.25) (layer "F.Cu") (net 14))
 (segment (start 49.275 -11.1) (end 48.825 -10.65) (width 0.25) (layer "F.Cu") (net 14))
 (segment (start 49.275 -12.152) (end 49.275 -11.1) (width 0.25) (layer "F.Cu") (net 14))
 (segment (start 48.825 -10.65) (end 48.825 -6.075) (width 0.25) (layer "F.Cu") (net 14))
 (segment (start 49.275 -13.848) (end 49.275 -14.725) (width 0.25) (layer "F.Cu") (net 15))
 (segment (start 49.275 -14.725) (end 48.875 -15.125) (width 0.25) (layer "F.Cu") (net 15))
 (segment (start 36.875 -22.025) (end 28.698 -13.848) (width 0.25) (layer "F.Cu") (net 15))
 (segment (start 28.698 -13.848) (end 26.875 -13.848) (width 0.25) (layer "F.Cu") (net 15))
 (segment (start 48.875 -15.125) (end 48.875 -20.3) (width 0.25) (layer "F.Cu") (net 15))
 (segment (start 48.875 -20.3) (end 47.15 -22.025) (width 0.25) (layer "F.Cu") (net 15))
 (segment (start 47.15 -22.025) (end 36.875 -22.025) (width 0.25) (layer "F.Cu") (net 15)))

